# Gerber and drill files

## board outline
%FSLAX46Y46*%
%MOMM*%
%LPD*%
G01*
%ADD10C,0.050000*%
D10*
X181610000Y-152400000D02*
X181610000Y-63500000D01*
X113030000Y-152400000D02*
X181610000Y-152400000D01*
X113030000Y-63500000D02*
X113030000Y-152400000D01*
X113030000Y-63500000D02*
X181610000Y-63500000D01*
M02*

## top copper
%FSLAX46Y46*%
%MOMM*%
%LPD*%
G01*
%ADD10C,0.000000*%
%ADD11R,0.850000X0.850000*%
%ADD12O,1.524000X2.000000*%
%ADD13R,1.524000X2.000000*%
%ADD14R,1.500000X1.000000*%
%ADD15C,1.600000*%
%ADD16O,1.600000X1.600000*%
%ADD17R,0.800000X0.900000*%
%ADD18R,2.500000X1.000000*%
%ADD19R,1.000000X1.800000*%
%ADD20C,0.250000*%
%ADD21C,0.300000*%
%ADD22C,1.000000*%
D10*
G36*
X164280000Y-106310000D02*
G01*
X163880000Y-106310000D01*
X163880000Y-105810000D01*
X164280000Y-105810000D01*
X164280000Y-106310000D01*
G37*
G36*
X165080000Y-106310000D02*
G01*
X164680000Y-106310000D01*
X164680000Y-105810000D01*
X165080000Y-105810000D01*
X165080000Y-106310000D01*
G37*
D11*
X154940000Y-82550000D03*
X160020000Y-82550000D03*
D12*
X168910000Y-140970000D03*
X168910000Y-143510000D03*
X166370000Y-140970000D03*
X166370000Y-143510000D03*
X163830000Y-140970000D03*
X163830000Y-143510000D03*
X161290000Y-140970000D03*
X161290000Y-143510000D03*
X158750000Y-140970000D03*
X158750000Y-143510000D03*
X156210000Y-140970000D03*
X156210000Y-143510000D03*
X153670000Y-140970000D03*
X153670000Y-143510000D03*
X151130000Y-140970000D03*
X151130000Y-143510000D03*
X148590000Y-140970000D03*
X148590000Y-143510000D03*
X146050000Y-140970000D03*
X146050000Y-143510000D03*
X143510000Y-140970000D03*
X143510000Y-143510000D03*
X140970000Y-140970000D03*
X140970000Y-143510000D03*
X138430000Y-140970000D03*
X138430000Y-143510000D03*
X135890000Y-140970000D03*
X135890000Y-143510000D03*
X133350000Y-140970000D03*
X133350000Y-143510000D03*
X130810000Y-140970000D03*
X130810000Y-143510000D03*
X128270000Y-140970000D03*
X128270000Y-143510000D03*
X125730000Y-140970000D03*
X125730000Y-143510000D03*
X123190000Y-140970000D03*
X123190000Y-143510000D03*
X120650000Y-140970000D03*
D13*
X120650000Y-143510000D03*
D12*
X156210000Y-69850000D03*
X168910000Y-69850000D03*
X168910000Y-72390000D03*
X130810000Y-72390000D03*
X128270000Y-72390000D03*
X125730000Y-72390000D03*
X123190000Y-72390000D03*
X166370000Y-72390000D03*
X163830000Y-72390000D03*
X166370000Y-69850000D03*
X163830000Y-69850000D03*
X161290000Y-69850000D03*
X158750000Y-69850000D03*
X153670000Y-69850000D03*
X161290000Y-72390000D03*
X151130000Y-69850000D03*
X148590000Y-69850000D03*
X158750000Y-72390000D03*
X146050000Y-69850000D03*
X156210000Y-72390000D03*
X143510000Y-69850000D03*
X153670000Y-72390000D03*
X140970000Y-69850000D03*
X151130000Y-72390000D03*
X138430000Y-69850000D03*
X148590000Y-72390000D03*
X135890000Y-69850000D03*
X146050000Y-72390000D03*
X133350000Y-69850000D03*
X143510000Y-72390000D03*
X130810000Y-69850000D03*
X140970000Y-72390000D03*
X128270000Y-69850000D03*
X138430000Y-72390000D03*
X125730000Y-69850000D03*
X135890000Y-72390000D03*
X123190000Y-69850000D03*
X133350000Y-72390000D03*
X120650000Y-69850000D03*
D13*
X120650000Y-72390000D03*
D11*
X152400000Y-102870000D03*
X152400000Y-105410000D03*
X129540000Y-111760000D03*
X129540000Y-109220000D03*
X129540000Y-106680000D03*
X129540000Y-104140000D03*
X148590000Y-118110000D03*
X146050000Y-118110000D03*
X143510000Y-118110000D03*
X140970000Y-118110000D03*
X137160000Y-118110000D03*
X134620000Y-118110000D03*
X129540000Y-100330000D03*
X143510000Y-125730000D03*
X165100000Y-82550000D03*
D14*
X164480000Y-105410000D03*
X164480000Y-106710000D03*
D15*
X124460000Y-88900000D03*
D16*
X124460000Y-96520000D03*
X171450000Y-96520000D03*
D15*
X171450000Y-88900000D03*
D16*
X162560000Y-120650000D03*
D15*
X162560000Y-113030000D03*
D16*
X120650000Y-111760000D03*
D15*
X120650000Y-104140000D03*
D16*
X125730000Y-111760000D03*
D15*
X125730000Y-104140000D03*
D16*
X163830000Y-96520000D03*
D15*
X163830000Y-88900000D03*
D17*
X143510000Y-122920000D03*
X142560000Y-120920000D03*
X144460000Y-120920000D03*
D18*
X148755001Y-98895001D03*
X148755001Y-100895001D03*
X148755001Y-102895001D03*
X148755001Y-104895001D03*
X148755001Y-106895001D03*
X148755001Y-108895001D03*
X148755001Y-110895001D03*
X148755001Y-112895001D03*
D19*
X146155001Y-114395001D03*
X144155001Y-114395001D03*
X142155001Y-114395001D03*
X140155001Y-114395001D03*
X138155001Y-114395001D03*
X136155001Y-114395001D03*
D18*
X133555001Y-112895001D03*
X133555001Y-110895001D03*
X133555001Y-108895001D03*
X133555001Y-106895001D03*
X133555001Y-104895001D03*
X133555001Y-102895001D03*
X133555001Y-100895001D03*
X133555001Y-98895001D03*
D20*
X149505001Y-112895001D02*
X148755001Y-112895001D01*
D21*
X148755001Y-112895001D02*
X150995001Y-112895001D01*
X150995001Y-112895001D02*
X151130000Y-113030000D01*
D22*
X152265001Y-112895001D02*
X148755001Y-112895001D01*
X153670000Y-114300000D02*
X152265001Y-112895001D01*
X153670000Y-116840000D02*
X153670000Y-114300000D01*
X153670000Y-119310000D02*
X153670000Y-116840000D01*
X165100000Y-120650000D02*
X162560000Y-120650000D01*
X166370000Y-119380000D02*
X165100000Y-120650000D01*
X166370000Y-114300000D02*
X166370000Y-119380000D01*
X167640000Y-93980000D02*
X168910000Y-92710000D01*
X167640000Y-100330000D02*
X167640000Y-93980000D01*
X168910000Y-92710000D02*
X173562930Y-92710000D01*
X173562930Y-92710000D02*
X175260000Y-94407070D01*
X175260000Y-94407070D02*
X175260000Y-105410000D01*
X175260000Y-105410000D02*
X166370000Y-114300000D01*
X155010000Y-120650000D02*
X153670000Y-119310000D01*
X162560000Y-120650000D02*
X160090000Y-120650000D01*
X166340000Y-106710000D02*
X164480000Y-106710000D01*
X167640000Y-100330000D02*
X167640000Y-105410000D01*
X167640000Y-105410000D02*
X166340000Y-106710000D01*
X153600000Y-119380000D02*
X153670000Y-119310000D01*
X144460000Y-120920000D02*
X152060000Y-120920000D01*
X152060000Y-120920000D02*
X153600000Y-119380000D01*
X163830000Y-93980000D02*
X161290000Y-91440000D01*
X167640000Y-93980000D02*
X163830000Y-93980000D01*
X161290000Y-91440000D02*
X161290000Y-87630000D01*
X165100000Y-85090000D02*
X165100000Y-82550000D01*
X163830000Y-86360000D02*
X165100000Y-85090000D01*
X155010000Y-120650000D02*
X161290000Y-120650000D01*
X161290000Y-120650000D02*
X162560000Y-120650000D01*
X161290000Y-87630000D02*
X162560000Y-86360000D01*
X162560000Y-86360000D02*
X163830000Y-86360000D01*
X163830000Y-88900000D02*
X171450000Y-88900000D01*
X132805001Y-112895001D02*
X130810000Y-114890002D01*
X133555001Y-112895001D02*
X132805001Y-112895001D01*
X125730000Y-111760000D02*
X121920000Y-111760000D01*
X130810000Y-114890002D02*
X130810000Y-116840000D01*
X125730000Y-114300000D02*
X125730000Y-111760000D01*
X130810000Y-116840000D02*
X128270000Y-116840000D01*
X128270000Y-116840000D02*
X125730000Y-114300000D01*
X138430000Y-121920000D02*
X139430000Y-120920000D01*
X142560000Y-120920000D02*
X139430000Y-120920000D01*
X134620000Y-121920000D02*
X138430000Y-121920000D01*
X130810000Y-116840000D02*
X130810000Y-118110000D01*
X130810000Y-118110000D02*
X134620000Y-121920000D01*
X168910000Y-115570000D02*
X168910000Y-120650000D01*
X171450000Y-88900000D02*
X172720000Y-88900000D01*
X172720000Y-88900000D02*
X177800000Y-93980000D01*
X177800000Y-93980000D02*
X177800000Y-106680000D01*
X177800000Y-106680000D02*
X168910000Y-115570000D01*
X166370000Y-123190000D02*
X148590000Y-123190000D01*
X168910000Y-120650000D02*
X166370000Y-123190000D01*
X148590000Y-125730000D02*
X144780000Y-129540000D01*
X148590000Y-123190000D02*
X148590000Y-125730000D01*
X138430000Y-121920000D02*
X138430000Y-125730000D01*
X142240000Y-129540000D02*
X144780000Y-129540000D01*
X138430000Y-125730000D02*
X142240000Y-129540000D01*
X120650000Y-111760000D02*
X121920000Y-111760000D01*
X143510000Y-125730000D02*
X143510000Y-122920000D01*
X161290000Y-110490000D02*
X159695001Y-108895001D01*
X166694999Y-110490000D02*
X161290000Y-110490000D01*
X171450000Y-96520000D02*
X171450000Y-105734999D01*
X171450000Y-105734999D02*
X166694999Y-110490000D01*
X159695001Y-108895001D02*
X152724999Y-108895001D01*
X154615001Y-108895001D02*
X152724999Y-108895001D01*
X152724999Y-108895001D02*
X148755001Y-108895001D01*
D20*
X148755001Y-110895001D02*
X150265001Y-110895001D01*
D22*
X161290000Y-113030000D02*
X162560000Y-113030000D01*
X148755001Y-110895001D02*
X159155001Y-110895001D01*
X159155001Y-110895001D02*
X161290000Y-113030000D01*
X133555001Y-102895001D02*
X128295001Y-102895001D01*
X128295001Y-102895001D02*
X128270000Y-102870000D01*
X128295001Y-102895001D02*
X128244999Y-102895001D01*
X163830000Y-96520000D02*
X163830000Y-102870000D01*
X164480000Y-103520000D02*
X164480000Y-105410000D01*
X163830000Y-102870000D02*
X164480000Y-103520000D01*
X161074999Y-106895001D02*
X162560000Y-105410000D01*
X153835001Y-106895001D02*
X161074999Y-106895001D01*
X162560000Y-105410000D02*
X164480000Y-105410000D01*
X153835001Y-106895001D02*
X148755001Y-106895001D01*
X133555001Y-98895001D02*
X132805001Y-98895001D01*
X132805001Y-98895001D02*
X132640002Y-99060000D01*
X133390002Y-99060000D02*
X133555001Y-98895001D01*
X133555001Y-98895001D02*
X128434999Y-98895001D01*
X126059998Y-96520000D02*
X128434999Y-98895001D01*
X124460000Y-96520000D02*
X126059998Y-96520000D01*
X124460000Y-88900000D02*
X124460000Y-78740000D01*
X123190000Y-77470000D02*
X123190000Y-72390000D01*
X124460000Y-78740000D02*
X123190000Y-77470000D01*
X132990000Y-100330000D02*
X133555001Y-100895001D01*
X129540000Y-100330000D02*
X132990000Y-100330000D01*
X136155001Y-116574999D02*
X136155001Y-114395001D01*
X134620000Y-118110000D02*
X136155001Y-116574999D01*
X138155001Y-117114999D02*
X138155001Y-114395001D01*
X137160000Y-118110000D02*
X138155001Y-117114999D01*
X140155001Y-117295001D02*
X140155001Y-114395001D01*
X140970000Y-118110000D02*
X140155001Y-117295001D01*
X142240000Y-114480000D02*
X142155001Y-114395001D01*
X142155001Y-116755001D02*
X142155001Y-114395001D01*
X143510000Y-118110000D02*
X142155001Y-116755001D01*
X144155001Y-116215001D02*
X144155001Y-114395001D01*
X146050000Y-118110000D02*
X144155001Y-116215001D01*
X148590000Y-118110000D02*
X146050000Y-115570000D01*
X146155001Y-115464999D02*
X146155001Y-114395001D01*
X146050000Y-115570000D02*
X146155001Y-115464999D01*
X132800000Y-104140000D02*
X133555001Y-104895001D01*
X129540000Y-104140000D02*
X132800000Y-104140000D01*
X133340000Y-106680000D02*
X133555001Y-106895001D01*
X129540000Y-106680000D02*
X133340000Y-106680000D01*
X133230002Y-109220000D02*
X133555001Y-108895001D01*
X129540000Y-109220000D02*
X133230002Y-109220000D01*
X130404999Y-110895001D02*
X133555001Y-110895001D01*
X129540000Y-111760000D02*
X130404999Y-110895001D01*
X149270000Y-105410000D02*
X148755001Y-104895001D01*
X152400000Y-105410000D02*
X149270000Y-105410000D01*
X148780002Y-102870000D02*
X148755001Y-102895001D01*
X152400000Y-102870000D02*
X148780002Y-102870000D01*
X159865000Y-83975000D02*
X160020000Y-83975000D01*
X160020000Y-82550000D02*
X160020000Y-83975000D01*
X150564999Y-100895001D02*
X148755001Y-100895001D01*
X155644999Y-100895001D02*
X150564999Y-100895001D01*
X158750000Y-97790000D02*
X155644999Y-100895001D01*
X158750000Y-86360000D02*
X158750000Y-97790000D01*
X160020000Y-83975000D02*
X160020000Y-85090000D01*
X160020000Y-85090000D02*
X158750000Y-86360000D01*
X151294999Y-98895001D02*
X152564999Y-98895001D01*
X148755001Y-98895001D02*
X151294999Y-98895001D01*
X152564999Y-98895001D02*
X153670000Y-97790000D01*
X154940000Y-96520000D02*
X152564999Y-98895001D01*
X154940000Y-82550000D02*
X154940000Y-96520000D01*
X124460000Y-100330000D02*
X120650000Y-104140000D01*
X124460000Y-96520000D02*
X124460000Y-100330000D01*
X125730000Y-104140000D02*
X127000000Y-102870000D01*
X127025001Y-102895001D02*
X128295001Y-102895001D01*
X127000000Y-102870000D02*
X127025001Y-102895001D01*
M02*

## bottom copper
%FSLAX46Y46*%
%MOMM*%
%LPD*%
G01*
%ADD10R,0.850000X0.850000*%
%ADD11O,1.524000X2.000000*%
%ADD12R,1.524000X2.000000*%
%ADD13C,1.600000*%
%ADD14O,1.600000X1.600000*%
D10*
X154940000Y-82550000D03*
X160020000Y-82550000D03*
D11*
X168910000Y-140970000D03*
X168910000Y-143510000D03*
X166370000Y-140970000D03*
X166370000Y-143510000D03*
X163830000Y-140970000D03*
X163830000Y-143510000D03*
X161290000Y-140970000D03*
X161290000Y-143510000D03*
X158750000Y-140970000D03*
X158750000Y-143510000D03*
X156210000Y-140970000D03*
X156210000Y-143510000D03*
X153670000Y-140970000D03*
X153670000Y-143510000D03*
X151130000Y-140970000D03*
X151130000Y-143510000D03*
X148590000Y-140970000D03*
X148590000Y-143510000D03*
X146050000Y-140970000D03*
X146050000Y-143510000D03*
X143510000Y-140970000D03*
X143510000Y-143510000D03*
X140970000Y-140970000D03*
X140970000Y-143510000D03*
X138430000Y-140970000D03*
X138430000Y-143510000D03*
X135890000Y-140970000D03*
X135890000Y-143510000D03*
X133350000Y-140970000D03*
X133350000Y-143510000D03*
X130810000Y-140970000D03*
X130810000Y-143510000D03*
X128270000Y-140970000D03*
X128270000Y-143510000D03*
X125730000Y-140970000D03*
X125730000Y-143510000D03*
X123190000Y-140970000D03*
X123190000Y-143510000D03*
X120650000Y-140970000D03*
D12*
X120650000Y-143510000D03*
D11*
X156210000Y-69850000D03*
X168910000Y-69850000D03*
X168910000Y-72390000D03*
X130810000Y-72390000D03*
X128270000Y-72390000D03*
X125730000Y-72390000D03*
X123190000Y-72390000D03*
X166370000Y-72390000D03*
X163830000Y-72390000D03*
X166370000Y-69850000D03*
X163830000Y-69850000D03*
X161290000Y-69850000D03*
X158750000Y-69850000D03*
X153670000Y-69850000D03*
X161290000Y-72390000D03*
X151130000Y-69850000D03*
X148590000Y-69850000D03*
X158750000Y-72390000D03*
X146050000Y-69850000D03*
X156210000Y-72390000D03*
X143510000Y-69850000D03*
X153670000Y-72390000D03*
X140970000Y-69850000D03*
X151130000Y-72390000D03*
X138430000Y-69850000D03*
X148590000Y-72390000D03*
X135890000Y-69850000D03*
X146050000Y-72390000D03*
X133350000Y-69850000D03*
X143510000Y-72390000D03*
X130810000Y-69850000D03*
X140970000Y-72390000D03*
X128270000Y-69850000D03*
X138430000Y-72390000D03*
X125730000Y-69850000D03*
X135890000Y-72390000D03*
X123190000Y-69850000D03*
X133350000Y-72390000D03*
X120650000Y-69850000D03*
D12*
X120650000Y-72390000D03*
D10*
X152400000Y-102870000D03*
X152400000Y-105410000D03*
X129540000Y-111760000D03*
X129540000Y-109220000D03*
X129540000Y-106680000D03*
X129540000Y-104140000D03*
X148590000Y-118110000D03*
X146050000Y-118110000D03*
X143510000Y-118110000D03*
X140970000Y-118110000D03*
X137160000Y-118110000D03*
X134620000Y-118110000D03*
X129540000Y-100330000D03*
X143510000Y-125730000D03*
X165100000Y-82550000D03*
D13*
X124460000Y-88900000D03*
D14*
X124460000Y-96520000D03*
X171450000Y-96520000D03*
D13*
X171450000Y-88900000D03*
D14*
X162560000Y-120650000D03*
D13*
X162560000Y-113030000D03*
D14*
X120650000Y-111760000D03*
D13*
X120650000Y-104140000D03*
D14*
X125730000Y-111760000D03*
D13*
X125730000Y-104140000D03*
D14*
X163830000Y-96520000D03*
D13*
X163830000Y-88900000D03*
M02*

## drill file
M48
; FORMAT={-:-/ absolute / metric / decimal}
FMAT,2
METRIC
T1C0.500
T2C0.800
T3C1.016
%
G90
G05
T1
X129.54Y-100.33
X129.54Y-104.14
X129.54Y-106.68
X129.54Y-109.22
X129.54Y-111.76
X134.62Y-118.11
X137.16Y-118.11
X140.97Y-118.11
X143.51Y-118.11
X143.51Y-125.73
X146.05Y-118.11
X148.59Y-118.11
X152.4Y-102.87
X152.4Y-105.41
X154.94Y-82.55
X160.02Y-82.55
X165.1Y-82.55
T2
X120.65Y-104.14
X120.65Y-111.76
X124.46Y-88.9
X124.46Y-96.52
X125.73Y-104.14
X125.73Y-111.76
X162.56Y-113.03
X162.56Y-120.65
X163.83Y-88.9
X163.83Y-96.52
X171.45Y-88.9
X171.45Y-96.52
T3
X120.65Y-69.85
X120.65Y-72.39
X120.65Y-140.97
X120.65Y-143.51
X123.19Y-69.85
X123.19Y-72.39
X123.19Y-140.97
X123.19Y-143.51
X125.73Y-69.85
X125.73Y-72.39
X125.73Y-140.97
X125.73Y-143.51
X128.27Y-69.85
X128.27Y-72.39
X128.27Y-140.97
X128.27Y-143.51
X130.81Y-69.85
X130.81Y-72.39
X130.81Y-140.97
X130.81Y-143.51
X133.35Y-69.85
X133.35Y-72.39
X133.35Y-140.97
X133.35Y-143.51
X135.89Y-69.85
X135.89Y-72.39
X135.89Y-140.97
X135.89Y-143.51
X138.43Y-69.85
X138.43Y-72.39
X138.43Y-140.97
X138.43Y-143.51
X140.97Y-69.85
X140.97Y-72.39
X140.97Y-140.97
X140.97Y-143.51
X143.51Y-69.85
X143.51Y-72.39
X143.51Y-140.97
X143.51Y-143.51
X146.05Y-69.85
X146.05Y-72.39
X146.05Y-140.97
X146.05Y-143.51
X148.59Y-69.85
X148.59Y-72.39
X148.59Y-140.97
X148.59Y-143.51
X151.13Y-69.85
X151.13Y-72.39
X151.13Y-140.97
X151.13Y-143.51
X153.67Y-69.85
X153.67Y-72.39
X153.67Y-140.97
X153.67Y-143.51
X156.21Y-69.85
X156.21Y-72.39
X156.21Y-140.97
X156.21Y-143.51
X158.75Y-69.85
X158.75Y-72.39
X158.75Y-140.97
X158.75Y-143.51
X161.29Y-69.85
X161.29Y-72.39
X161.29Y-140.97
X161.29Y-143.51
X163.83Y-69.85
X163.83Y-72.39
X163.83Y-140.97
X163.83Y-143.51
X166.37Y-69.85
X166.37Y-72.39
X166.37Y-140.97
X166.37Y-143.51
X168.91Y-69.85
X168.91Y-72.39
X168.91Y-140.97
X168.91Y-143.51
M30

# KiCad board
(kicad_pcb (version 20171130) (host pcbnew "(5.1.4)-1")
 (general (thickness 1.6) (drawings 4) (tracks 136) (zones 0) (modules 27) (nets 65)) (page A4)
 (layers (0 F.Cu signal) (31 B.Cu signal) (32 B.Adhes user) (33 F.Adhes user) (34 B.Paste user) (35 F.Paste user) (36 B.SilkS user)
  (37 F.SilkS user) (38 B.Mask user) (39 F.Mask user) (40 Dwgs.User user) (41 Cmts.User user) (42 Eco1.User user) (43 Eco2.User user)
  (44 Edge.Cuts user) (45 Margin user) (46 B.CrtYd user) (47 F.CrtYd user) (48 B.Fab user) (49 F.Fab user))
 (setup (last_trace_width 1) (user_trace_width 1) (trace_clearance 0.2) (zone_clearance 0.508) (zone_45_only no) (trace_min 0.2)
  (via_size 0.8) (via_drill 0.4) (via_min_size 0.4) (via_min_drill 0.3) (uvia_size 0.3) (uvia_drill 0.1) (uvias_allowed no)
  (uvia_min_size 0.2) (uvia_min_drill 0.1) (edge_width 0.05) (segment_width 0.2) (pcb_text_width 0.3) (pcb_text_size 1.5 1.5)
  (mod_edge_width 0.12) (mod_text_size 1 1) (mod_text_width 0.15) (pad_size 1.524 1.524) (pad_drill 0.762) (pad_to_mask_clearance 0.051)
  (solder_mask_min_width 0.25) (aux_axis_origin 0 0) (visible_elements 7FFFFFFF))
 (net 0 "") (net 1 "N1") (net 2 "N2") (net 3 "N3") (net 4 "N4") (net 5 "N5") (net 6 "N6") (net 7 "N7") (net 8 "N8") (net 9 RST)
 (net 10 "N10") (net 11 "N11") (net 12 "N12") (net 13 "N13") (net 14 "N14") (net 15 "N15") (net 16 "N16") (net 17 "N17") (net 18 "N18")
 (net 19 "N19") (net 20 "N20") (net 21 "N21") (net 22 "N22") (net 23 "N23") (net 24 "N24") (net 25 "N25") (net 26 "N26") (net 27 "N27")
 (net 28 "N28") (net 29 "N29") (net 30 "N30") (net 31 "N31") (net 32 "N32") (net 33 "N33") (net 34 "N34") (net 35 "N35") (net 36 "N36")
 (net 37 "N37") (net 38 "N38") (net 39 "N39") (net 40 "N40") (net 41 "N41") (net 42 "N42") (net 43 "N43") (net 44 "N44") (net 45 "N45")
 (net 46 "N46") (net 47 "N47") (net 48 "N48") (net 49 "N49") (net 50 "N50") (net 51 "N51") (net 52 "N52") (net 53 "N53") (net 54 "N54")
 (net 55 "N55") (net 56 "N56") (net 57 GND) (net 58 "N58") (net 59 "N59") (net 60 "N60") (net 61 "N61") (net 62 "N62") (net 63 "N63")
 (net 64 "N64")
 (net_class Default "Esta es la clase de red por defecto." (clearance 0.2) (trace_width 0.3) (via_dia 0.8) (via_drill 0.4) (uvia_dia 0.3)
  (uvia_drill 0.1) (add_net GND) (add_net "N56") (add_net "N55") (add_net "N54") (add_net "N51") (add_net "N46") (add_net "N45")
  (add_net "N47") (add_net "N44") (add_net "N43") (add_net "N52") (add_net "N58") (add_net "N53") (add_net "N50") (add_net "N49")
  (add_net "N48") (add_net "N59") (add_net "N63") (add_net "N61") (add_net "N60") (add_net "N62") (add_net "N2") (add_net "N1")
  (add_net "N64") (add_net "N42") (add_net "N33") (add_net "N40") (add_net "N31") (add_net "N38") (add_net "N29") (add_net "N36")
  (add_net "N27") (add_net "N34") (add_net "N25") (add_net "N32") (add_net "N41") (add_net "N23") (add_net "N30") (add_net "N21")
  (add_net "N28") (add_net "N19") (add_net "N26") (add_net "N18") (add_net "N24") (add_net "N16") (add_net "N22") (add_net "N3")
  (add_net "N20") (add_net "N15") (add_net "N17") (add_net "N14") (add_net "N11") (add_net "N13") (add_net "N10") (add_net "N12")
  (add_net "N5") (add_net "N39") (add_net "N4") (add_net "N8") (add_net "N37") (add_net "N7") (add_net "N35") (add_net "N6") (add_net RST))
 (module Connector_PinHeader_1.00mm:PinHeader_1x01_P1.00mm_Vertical (layer F.Cu) (at 154.94 82.55)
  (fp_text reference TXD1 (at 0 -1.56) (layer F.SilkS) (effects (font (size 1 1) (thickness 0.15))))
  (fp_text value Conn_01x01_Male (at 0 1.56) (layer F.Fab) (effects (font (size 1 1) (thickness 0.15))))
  (pad 1 thru_hole rect (at 0 0) (size 0.85 0.85) (drill 0.5) (layers *.Cu *.Mask) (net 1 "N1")))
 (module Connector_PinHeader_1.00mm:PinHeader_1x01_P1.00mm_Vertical (layer F.Cu) (at 160.02 82.55)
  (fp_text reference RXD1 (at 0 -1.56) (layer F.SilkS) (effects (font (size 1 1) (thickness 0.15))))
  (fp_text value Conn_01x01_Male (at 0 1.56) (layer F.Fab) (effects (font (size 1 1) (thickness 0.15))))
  (pad 1 thru_hole rect (at 0 0) (size 0.85 0.85) (drill 0.5) (layers *.Cu *.Mask) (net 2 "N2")))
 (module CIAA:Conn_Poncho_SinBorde (layer F.Cu) (at 120.65 72.39 90)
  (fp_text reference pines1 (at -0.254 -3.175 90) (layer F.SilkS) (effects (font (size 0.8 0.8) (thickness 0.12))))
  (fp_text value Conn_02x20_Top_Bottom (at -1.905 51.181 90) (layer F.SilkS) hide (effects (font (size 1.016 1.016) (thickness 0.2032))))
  (pad 80 thru_hole oval (at -68.58 48.26) (size 1.524 2) (drill 1.016) (layers *.Cu *.Mask F.SilkS))
  (pad 79 thru_hole oval (at -71.12 48.26) (size 1.524 2) (drill 1.016) (layers *.Cu *.Mask F.SilkS))
  (pad 78 thru_hole oval (at -68.58 45.72) (size 1.524 2) (drill 1.016) (layers *.Cu *.Mask F.SilkS))
  (pad 77 thru_hole oval (at -71.12 45.72) (size 1.524 2) (drill 1.016) (layers *.Cu *.Mask F.SilkS))
  (pad 76 thru_hole oval (at -68.58 43.18) (size 1.524 2) (drill 1.016) (layers *.Cu *.Mask F.SilkS))
  (pad 75 thru_hole oval (at -71.12 43.18) (size 1.524 2) (drill 1.016) (layers *.Cu *.Mask F.SilkS))
  (pad 74 thru_hole oval (at -68.58 40.64) (size 1.524 2) (drill 1.016) (layers *.Cu *.Mask F.SilkS))
  (pad 73 thru_hole oval (at -71.12 40.64) (size 1.524 2) (drill 1.016) (layers *.Cu *.Mask F.SilkS))
  (pad 72 thru_hole oval (at -68.58 38.1) (size 1.524 2) (drill 1.016) (layers *.Cu *.Mask F.SilkS))
  (pad 71 thru_hole oval (at -71.12 38.1) (size 1.524 2) (drill 1.016) (layers *.Cu *.Mask F.SilkS))
  (pad 70 thru_hole oval (at -68.58 35.56) (size 1.524 2) (drill 1.016) (layers *.Cu *.Mask F.SilkS))
  (pad 69 thru_hole oval (at -71.12 35.56) (size 1.524 2) (drill 1.016) (layers *.Cu *.Mask F.SilkS))
  (pad 68 thru_hole oval (at -68.58 33.02) (size 1.524 2) (drill 1.016) (layers *.Cu *.Mask F.SilkS))
  (pad 67 thru_hole oval (at -71.12 33.02) (size 1.524 2) (drill 1.016) (layers *.Cu *.Mask F.SilkS))
  (pad 66 thru_hole oval (at -68.58 30.48) (size 1.524 2) (drill 1.016) (layers *.Cu *.Mask F.SilkS))
  (pad 65 thru_hole oval (at -71.12 30.48) (size 1.524 2) (drill 1.016) (layers *.Cu *.Mask F.SilkS))
  (pad 64 thru_hole oval (at -68.58 27.94) (size 1.524 2) (drill 1.016) (layers *.Cu *.Mask F.SilkS))
  (pad 63 thru_hole oval (at -71.12 27.94) (size 1.524 2) (drill 1.016) (layers *.Cu *.Mask F.SilkS))
  (pad 62 thru_hole oval (at -68.58 25.4) (size 1.524 2) (drill 1.016) (layers *.Cu *.Mask F.SilkS))
  (pad 61 thru_hole oval (at -71.12 25.4) (size 1.524 2) (drill 1.016) (layers *.Cu *.Mask F.SilkS))
  (pad 60 thru_hole oval (at -68.58 22.86) (size 1.524 2) (drill 1.016) (layers *.Cu *.Mask F.SilkS))
  (pad 59 thru_hole oval (at -71.12 22.86) (size 1.524 2) (drill 1.016) (layers *.Cu *.Mask F.SilkS))
  (pad 58 thru_hole oval (at -68.58 20.32) (size 1.524 2) (drill 1.016) (layers *.Cu *.Mask F.SilkS))
  (pad 57 thru_hole oval (at -71.12 20.32) (size 1.524 2) (drill 1.016) (layers *.Cu *.Mask F.SilkS))
  (pad 56 thru_hole oval (at -68.58 17.78) (size 1.524 2) (drill 1.016) (layers *.Cu *.Mask F.SilkS))
  (pad 55 thru_hole oval (at -71.12 17.78) (size 1.524 2) (drill 1.016) (layers *.Cu *.Mask F.SilkS))
  (pad 54 thru_hole oval (at -68.58 15.24) (size 1.524 2) (drill 1.016) (layers *.Cu *.Mask F.SilkS))
  (pad 53 thru_hole oval (at -71.12 15.24) (size 1.524 2) (drill 1.016) (layers *.Cu *.Mask F.SilkS))
  (pad 52 thru_hole oval (at -68.58 12.7) (size 1.524 2) (drill 1.016) (layers *.Cu *.Mask F.SilkS))
  (pad 51 thru_hole oval (at -71.12 12.7) (size 1.524 2) (drill 1.016) (layers *.Cu *.Mask F.SilkS))
  (pad 50 thru_hole oval (at -68.58 10.16) (size 1.524 2) (drill 1.016) (layers *.Cu *.Mask F.SilkS))
  (pad 49 thru_hole oval (at -71.12 10.16) (size 1.524 2) (drill 1.016) (layers *.Cu *.Mask F.SilkS))
  (pad 48 thru_hole oval (at -68.58 7.62) (size 1.524 2) (drill 1.016) (layers *.Cu *.Mask F.SilkS))
  (pad 47 thru_hole oval (at -71.12 7.62) (size 1.524 2) (drill 1.016) (layers *.Cu *.Mask F.SilkS))
  (pad 46 thru_hole oval (at -68.58 5.08) (size 1.524 2) (drill 1.016) (layers *.Cu *.Mask F.SilkS))
  (pad 45 thru_hole oval (at -71.12 5.08) (size 1.524 2) (drill 1.016) (layers *.Cu *.Mask F.SilkS))
  (pad 44 thru_hole oval (at -68.58 2.54) (size 1.524 2) (drill 1.016) (layers *.Cu *.Mask F.SilkS))
  (pad 43 thru_hole oval (at -71.12 2.54) (size 1.524 2) (drill 1.016) (layers *.Cu *.Mask F.SilkS))
  (pad 42 thru_hole oval (at -68.58 0) (size 1.524 2) (drill 1.016) (layers *.Cu *.Mask F.SilkS))
  (pad 41 thru_hole rect (at -71.12 0) (size 1.524 2) (drill 1.016) (layers *.Cu *.Mask F.SilkS))
  (pad 30 thru_hole oval (at 2.54 35.56) (size 1.524 2) (drill 1.016) (layers *.Cu *.Mask F.SilkS) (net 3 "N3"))
  (pad 40 thru_hole oval (at 2.54 48.26) (size 1.524 2) (drill 1.016) (layers *.Cu *.Mask F.SilkS) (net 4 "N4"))
  (pad 39 thru_hole oval (at 0 48.26) (size 1.524 2) (drill 1.016) (layers *.Cu *.Mask F.SilkS) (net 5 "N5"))
  (pad 9 thru_hole oval (at 0 10.16) (size 1.524 2) (drill 1.016) (layers *.Cu *.Mask F.SilkS) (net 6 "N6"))
  (pad 7 thru_hole oval (at 0 7.62) (size 1.524 2) (drill 1.016) (layers *.Cu *.Mask F.SilkS) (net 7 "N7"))
  (pad 5 thru_hole oval (at 0 5.08) (size 1.524 2) (drill 1.016) (layers *.Cu *.Mask F.SilkS) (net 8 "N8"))
  (pad 3 thru_hole oval (at 0 2.54) (size 1.524 2) (drill 1.016) (layers *.Cu *.Mask F.SilkS) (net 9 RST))
  (pad 37 thru_hole oval (at 0 45.72) (size 1.524 2) (drill 1.016) (layers *.Cu *.Mask F.SilkS) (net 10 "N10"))
  (pad 35 thru_hole oval (at 0 43.18) (size 1.524 2) (drill 1.016) (layers *.Cu *.Mask F.SilkS) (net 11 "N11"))
  (pad 38 thru_hole oval (at 2.54 45.72) (size 1.524 2) (drill 1.016) (layers *.Cu *.Mask F.SilkS) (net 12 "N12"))
  (pad 36 thru_hole oval (at 2.54 43.18) (size 1.524 2) (drill 1.016) (layers *.Cu *.Mask F.SilkS) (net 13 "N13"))
  (pad 34 thru_hole oval (at 2.54 40.64) (size 1.524 2) (drill 1.016) (layers *.Cu *.Mask F.SilkS) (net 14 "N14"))
  (pad 32 thru_hole oval (at 2.54 38.1) (size 1.524 2) (drill 1.016) (layers *.Cu *.Mask F.SilkS) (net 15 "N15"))
  (pad 28 thru_hole oval (at 2.54 33.02) (size 1.524 2) (drill 1.016) (layers *.Cu *.Mask F.SilkS) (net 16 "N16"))
  (pad 33 thru_hole oval (at 0 40.64) (size 1.524 2) (drill 1.016) (layers *.Cu *.Mask F.SilkS) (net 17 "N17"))
  (pad 26 thru_hole oval (at 2.54 30.48) (size 1.524 2) (drill 1.016) (layers *.Cu *.Mask F.SilkS) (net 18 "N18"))
  (pad 24 thru_hole oval (at 2.54 27.94) (size 1.524 2) (drill 1.016) (layers *.Cu *.Mask F.SilkS) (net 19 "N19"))
  (pad 31 thru_hole oval (at 0 38.1) (size 1.524 2) (drill 1.016) (layers *.Cu *.Mask F.SilkS) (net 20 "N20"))
  (pad 22 thru_hole oval (at 2.54 25.4) (size 1.524 2) (drill 1.016) (layers *.Cu *.Mask F.SilkS) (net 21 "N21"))
  (pad 29 thru_hole oval (at 0 35.56) (size 1.524 2) (drill 1.016) (layers *.Cu *.Mask F.SilkS) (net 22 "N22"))
  (pad 20 thru_hole oval (at 2.54 22.86) (size 1.524 2) (drill 1.016) (layers *.Cu *.Mask F.SilkS) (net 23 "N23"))
  (pad 27 thru_hole oval (at 0 33.02) (size 1.524 2) (drill 1.016) (layers *.Cu *.Mask F.SilkS) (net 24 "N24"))
  (pad 18 thru_hole oval (at 2.54 20.32) (size 1.524 2) (drill 1.016) (layers *.Cu *.Mask F.SilkS) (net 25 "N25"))
  (pad 25 thru_hole oval (at 0 30.48) (size 1.524 2) (drill 1.016) (layers *.Cu *.Mask F.SilkS) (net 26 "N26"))
  (pad 16 thru_hole oval (at 2.54 17.78) (size 1.524 2) (drill 1.016) (layers *.Cu *.Mask F.SilkS) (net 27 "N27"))
  (pad 23 thru_hole oval (at 0 27.94) (size 1.524 2) (drill 1.016) (layers *.Cu *.Mask F.SilkS) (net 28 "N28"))
  (pad 14 thru_hole oval (at 2.54 15.24) (size 1.524 2) (drill 1.016) (layers *.Cu *.Mask F.SilkS) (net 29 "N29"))
  (pad 21 thru_hole oval (at 0 25.4) (size 1.524 2) (drill 1.016) (layers *.Cu *.Mask F.SilkS) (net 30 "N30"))
  (pad 12 thru_hole oval (at 2.54 12.7) (size 1.524 2) (drill 1.016) (layers *.Cu *.Mask F.SilkS) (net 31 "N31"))
  (pad 19 thru_hole oval (at 0 22.86) (size 1.524 2) (drill 1.016) (layers *.Cu *.Mask F.SilkS) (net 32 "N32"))
  (pad 10 thru_hole oval (at 2.54 10.16) (size 1.524 2) (drill 1.016) (layers *.Cu *.Mask F.SilkS) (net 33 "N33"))
  (pad 17 thru_hole oval (at 0 20.32) (size 1.524 2) (drill 1.016) (layers *.Cu *.Mask F.SilkS) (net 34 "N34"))
  (pad 8 thru_hole oval (at 2.54 7.62) (size 1.524 2) (drill 1.016) (layers *.Cu *.Mask F.SilkS) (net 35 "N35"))
  (pad 15 thru_hole oval (at 0 17.78) (size 1.524 2) (drill 1.016) (layers *.Cu *.Mask F.SilkS) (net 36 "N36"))
  (pad 6 thru_hole oval (at 2.54 5.08) (size 1.524 2) (drill 1.016) (layers *.Cu *.Mask F.SilkS) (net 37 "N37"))
  (pad 13 thru_hole oval (at 0 15.24) (size 1.524 2) (drill 1.016) (layers *.Cu *.Mask F.SilkS) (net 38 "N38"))
  (pad 4 thru_hole oval (at 2.54 2.54) (size 1.524 2) (drill 1.016) (layers *.Cu *.Mask F.SilkS) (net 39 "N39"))
  (pad 11 thru_hole oval (at 0 12.7) (size 1.524 2) (drill 1.016) (layers *.Cu *.Mask F.SilkS) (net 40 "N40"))
  (pad 2 thru_hole oval (at 2.54 0) (size 1.524 2) (drill 1.016) (layers *.Cu *.Mask F.SilkS) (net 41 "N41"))
  (pad 1 thru_hole rect (at 0 0) (size 1.524 2) (drill 1.016) (layers *.Cu *.Mask F.SilkS) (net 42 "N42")))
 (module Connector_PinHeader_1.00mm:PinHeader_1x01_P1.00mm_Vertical (layer F.Cu) (at 152.4 102.87)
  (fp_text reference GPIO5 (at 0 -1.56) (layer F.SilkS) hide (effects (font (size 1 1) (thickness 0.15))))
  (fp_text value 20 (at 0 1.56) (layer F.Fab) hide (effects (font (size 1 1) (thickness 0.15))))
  (pad 1 thru_hole rect (at 0 0) (size 0.85 0.85) (drill 0.5) (layers *.Cu *.Mask) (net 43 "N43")))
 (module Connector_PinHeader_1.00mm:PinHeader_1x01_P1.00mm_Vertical (layer F.Cu) (at 152.4 105.41)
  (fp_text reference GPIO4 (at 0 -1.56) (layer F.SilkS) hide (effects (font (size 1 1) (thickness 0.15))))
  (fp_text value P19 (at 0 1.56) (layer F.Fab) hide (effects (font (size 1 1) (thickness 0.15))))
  (pad 1 thru_hole rect (at 0 0) (size 0.85 0.85) (drill 0.5) (layers *.Cu *.Mask) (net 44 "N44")))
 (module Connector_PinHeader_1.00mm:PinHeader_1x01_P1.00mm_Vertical (layer F.Cu) (at 129.54 111.76)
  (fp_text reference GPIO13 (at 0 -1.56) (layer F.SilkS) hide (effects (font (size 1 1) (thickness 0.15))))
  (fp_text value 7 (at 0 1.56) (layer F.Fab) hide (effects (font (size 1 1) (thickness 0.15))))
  (pad 1 thru_hole rect (at 0 0) (size 0.85 0.85) (drill 0.5) (layers *.Cu *.Mask) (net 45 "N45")))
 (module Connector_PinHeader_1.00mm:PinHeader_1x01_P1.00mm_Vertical (layer F.Cu) (at 129.54 109.22)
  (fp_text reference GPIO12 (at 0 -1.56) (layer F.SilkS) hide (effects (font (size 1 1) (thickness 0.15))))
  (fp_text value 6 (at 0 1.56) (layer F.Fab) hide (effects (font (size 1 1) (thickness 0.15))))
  (pad 1 thru_hole rect (at 0 0) (size 0.85 0.85) (drill 0.5) (layers *.Cu *.Mask) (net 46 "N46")))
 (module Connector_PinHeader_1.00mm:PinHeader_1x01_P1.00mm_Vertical (layer F.Cu) (at 129.54 106.68)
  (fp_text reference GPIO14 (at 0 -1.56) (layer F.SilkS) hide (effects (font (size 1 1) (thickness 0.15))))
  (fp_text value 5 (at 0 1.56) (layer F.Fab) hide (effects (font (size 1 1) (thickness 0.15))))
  (pad 1 thru_hole rect (at 0 0) (size 0.85 0.85) (drill 0.5) (layers *.Cu *.Mask) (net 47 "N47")))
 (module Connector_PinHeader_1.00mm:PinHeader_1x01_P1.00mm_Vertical (layer F.Cu) (at 129.54 104.14)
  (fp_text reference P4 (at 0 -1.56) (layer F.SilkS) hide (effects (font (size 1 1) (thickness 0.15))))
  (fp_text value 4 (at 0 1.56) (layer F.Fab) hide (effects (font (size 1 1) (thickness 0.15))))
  (pad 1 thru_hole rect (at 0 0) (size 0.85 0.85) (drill 0.5) (layers *.Cu *.Mask) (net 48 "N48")))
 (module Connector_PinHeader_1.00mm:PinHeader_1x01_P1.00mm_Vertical (layer F.Cu) (at 148.59 118.11)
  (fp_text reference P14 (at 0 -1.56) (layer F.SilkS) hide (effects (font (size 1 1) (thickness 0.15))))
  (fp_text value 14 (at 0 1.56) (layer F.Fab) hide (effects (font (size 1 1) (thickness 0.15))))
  (pad 1 thru_hole rect (at 0 0) (size 0.85 0.85) (drill 0.5) (layers *.Cu *.Mask) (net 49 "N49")))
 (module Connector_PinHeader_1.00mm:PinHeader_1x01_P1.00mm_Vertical (layer F.Cu) (at 146.05 118.11)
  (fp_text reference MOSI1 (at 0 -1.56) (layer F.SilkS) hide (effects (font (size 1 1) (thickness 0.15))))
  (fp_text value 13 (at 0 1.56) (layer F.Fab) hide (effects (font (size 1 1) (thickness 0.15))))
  (pad 1 thru_hole rect (at 0 0) (size 0.85 0.85) (drill 0.5) (layers *.Cu *.Mask) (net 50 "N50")))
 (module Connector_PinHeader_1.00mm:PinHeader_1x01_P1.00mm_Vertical (layer F.Cu) (at 143.51 118.11)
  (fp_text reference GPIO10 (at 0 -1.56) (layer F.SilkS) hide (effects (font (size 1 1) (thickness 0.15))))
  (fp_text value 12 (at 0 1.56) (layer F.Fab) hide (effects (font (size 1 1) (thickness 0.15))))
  (pad 1 thru_hole rect (at 0 0) (size 0.85 0.85) (drill 0.5) (layers *.Cu *.Mask) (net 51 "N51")))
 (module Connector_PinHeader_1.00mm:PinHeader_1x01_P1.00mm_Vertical (layer F.Cu) (at 140.97 118.11)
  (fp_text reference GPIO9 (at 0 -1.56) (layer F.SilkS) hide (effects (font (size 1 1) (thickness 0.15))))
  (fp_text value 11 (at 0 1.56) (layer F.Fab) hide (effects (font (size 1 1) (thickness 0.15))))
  (pad 1 thru_hole rect (at 0 0) (size 0.85 0.85) (drill 0.5) (layers *.Cu *.Mask) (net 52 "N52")))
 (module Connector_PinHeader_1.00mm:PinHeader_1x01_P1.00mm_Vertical (layer F.Cu) (at 137.16 118.11)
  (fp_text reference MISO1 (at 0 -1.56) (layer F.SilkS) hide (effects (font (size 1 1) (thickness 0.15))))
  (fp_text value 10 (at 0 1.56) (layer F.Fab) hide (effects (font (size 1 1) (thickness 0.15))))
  (pad 1 thru_hole rect (at 0 0) (size 0.85 0.85) (drill 0.5) (layers *.Cu *.Mask) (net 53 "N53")))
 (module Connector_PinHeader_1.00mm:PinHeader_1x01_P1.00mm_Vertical (layer F.Cu) (at 134.62 118.11)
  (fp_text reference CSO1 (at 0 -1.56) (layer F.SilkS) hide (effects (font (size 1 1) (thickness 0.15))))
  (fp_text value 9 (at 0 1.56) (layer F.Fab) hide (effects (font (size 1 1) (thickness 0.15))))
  (pad 1 thru_hole rect (at 0 0) (size 0.85 0.85) (drill 0.5) (layers *.Cu *.Mask) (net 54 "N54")))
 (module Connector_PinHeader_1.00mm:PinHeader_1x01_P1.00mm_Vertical (layer F.Cu) (at 129.54 100.33)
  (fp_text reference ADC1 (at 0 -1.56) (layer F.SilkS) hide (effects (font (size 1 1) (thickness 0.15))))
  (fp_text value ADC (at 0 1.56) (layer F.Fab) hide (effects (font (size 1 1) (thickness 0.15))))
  (pad 1 thru_hole rect (at 0 0) (size 0.85 0.85) (drill 0.5) (layers *.Cu *.Mask) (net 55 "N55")))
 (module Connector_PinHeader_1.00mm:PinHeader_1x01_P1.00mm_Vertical (layer F.Cu) (at 143.51 125.73 180)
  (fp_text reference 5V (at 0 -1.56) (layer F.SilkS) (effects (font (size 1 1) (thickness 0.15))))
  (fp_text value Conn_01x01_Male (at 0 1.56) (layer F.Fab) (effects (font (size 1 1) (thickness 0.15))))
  (pad 1 thru_hole rect (at 0 0 180) (size 0.85 0.85) (drill 0.5) (layers *.Cu *.Mask) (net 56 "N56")))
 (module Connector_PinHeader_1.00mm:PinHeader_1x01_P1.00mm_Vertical (layer F.Cu) (at 165.1 82.55)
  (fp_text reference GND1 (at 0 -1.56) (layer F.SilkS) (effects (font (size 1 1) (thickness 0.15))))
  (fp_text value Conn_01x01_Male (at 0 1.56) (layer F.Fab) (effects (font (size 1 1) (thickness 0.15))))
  (pad 1 thru_hole rect (at 0 0) (size 0.85 0.85) (drill 0.5) (layers *.Cu *.Mask) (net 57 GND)))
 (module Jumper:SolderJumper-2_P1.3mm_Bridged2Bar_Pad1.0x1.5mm (layer F.Cu) (at 164.48 106.06 90)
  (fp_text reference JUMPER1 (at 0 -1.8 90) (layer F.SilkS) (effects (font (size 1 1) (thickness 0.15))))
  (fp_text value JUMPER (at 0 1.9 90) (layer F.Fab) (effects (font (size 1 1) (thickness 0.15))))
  (fp_poly (pts (xy -0.25 -0.6) (xy 0.25 -0.6) (xy 0.25 -0.2) (xy -0.25 -0.2)) (layer F.Cu) (width 0))
  (fp_poly (pts (xy -0.25 0.2) (xy 0.25 0.2) (xy 0.25 0.6) (xy -0.25 0.6)) (layer F.Cu) (width 0))
  (pad 2 smd rect (at 0.65 0 90) (size 1 1.5) (layers F.Cu F.Mask) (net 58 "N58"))
  (pad 1 smd rect (at -0.65 0 90) (size 1 1.5) (layers F.Cu F.Mask) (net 57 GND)))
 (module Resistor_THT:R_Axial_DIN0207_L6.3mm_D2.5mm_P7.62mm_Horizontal (layer F.Cu) (at 124.46 88.9 270)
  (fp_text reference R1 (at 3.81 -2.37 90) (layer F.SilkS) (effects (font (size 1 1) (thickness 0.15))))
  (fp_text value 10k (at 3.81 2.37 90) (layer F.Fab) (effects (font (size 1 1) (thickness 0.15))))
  (pad 1 thru_hole circle (at 0 0 270) (size 1.6 1.6) (drill 0.8) (layers *.Cu *.Mask) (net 9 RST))
  (pad 2 thru_hole oval (at 7.62 0 270) (size 1.6 1.6) (drill 0.8) (layers *.Cu *.Mask) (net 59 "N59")))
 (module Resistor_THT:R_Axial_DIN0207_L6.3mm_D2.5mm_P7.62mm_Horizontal (layer F.Cu) (at 171.45 88.9 270)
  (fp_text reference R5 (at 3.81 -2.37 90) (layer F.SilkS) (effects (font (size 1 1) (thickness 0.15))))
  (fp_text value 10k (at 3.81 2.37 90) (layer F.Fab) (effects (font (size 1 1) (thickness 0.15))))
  (pad 2 thru_hole oval (at 7.62 0 270) (size 1.6 1.6) (drill 0.8) (layers *.Cu *.Mask) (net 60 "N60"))
  (pad 1 thru_hole circle (at 0 0 270) (size 1.6 1.6) (drill 0.8) (layers *.Cu *.Mask) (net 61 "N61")))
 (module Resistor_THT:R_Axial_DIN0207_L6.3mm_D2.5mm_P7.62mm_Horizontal (layer F.Cu) (at 162.56 113.03 270)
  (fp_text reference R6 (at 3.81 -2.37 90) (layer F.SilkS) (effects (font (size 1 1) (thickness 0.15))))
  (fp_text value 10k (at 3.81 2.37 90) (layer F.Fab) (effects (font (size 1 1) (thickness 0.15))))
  (pad 2 thru_hole oval (at 7.62 0 270) (size 1.6 1.6) (drill 0.8) (layers *.Cu *.Mask) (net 57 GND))
  (pad 1 thru_hole circle (at 0 0 270) (size 1.6 1.6) (drill 0.8) (layers *.Cu *.Mask) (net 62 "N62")))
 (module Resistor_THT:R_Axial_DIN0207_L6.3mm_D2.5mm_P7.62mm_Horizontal (layer F.Cu) (at 120.65 104.14 270)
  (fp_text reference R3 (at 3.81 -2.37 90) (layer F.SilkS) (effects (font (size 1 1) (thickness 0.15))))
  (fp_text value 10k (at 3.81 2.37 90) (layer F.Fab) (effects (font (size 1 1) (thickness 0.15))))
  (pad 2 thru_hole oval (at 7.62 0 270) (size 1.6 1.6) (drill 0.8) (layers *.Cu *.Mask) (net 61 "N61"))
  (pad 1 thru_hole circle (at 0 0 270) (size 1.6 1.6) (drill 0.8) (layers *.Cu *.Mask) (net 59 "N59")))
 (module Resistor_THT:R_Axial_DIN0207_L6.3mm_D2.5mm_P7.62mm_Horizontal (layer F.Cu) (at 125.73 104.14 270)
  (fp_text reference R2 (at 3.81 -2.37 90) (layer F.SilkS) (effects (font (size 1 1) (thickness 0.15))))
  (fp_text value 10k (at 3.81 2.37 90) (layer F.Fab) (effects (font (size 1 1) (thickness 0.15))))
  (pad 2 thru_hole oval (at 7.62 0 270) (size 1.6 1.6) (drill 0.8) (layers *.Cu *.Mask) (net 61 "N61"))
  (pad 1 thru_hole circle (at 0 0 270) (size 1.6 1.6) (drill 0.8) (layers *.Cu *.Mask) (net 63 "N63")))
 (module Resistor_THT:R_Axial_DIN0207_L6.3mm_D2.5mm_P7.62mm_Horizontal (layer F.Cu) (at 163.83 88.9 270)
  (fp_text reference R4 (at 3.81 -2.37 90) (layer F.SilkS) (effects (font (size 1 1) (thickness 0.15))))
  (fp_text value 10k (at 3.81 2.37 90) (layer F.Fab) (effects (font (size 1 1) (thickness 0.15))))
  (pad 2 thru_hole oval (at 7.62 0 270) (size 1.6 1.6) (drill 0.8) (layers *.Cu *.Mask) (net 58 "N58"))
  (pad 1 thru_hole circle (at 0 0 270) (size 1.6 1.6) (drill 0.8) (layers *.Cu *.Mask) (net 61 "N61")))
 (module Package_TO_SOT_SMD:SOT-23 (layer F.Cu) (at 143.51 121.92 270)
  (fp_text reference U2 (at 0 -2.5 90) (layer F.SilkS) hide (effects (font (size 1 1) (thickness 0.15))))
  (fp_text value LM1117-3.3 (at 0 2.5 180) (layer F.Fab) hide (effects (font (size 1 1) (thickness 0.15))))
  (pad 3 smd rect (at 1 0 270) (size 0.9 0.8) (layers F.Cu F.Paste F.Mask) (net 56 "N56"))
  (pad 2 smd rect (at -1 0.95 270) (size 0.9 0.8) (layers F.Cu F.Paste F.Mask) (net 61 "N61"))
  (pad 1 smd rect (at -1 -0.95 270) (size 0.9 0.8) (layers F.Cu F.Paste F.Mask) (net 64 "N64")))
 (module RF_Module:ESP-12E (layer F.Cu) (at 141.155001 102.395001)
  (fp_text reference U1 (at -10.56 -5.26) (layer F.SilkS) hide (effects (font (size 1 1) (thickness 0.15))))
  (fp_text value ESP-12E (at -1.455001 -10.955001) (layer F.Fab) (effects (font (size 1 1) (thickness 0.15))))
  (pad 22 smd rect (at 7.6 -3.5) (size 2.5 1) (layers F.Cu F.Paste F.Mask) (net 1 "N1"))
  (pad 21 smd rect (at 7.6 -1.5) (size 2.5 1) (layers F.Cu F.Paste F.Mask) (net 2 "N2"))
  (pad 20 smd rect (at 7.6 0.5) (size 2.5 1) (layers F.Cu F.Paste F.Mask) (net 43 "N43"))
  (pad 19 smd rect (at 7.6 2.5) (size 2.5 1) (layers F.Cu F.Paste F.Mask) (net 44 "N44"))
  (pad 18 smd rect (at 7.6 4.5) (size 2.5 1) (layers F.Cu F.Paste F.Mask) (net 58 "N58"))
  (pad 17 smd rect (at 7.6 6.5) (size 2.5 1) (layers F.Cu F.Paste F.Mask) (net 60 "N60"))
  (pad 16 smd rect (at 7.6 8.5) (size 2.5 1) (layers F.Cu F.Paste F.Mask) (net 62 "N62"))
  (pad 15 smd rect (at 7.6 10.5) (size 2.5 1) (layers F.Cu F.Paste F.Mask) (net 57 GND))
  (pad 14 smd rect (at 5 12) (size 1 1.8) (layers F.Cu F.Paste F.Mask) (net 49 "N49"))
  (pad 13 smd rect (at 3 12) (size 1 1.8) (layers F.Cu F.Paste F.Mask) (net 50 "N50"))
  (pad 12 smd rect (at 1 12) (size 1 1.8) (layers F.Cu F.Paste F.Mask) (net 51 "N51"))
  (pad 11 smd rect (at -1 12) (size 1 1.8) (layers F.Cu F.Paste F.Mask) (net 52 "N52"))
  (pad 10 smd rect (at -3 12) (size 1 1.8) (layers F.Cu F.Paste F.Mask) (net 53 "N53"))
  (pad 9 smd rect (at -5 12) (size 1 1.8) (layers F.Cu F.Paste F.Mask) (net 54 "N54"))
  (pad 8 smd rect (at -7.6 10.5) (size 2.5 1) (layers F.Cu F.Paste F.Mask) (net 61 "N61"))
  (pad 7 smd rect (at -7.6 8.5) (size 2.5 1) (layers F.Cu F.Paste F.Mask) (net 45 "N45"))
  (pad 6 smd rect (at -7.6 6.5) (size 2.5 1) (layers F.Cu F.Paste F.Mask) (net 46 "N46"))
  (pad 5 smd rect (at -7.6 4.5) (size 2.5 1) (layers F.Cu F.Paste F.Mask) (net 47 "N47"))
  (pad 4 smd rect (at -7.6 2.5) (size 2.5 1) (layers F.Cu F.Paste F.Mask) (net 48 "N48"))
  (pad 3 smd rect (at -7.6 0.5) (size 2.5 1) (layers F.Cu F.Paste F.Mask) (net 63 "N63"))
  (pad 2 smd rect (at -7.6 -1.5) (size 2.5 1) (layers F.Cu F.Paste F.Mask) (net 55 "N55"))
  (pad 1 smd rect (at -7.6 -3.5) (size 2.5 1) (layers F.Cu F.Paste F.Mask) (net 59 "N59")))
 (gr_line (start 181.61 152.4) (end 181.61 63.5) (layer Edge.Cuts) (width 0.05))
 (gr_line (start 113.03 152.4) (end 181.61 152.4) (layer Edge.Cuts) (width 0.05))
 (gr_line (start 113.03 63.5) (end 113.03 152.4) (layer Edge.Cuts) (width 0.05))
 (gr_line (start 113.03 63.5) (end 181.61 63.5) (layer Edge.Cuts) (width 0.05))
 (segment (start 149.505001 112.895001) (end 148.755001 112.895001) (width 0.25) (layer F.Cu) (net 57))
 (segment (start 148.755001 112.895001) (end 150.995001 112.895001) (width 0.3) (layer F.Cu) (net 57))
 (segment (start 150.995001 112.895001) (end 151.13 113.03) (width 0.3) (layer F.Cu) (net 57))
 (segment (start 152.265001 112.895001) (end 148.755001 112.895001) (width 1) (layer F.Cu) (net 57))
 (segment (start 153.67 114.3) (end 152.265001 112.895001) (width 1) (layer F.Cu) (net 57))
 (segment (start 153.67 116.84) (end 153.67 114.3) (width 1) (layer F.Cu) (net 57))
 (segment (start 153.67 119.31) (end 153.67 116.84) (width 1) (layer F.Cu) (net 57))
 (segment (start 165.1 120.65) (end 162.56 120.65) (width 1) (layer F.Cu) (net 57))
 (segment (start 166.37 119.38) (end 165.1 120.65) (width 1) (layer F.Cu) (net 57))
 (segment (start 166.37 114.3) (end 166.37 119.38) (width 1) (layer F.Cu) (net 57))
 (segment (start 167.64 93.98) (end 168.91 92.71) (width 1) (layer F.Cu) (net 57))
 (segment (start 167.64 100.33) (end 167.64 93.98) (width 1) (layer F.Cu) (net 57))
 (segment (start 168.91 92.71) (end 173.56293 92.71) (width 1) (layer F.Cu) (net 57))
 (segment (start 173.56293 92.71) (end 175.26 94.40707) (width 1) (layer F.Cu) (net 57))
 (segment (start 175.26 94.40707) (end 175.26 105.41) (width 1) (layer F.Cu) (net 57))
 (segment (start 175.26 105.41) (end 166.37 114.3) (width 1) (layer F.Cu) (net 57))
 (segment (start 155.01 120.65) (end 153.67 119.31) (width 1) (layer F.Cu) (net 57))
 (segment (start 162.56 120.65) (end 160.09 120.65) (width 1) (layer F.Cu) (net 57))
 (segment (start 166.34 106.71) (end 164.48 106.71) (width 1) (layer F.Cu) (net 57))
 (segment (start 167.64 100.33) (end 167.64 105.41) (width 1) (layer F.Cu) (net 57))
 (segment (start 167.64 105.41) (end 166.34 106.71) (width 1) (layer F.Cu) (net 57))
 (segment (start 153.6 119.38) (end 153.67 119.31) (width 1) (layer F.Cu) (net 57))
 (segment (start 144.46 120.92) (end 152.06 120.92) (width 1) (layer F.Cu) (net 57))
 (segment (start 152.06 120.92) (end 153.6 119.38) (width 1) (layer F.Cu) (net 57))
 (segment (start 163.83 93.98) (end 161.29 91.44) (width 1) (layer F.Cu) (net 57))
 (segment (start 167.64 93.98) (end 163.83 93.98) (width 1) (layer F.Cu) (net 57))
 (segment (start 161.29 91.44) (end 161.29 87.63) (width 1) (layer F.Cu) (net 57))
 (segment (start 165.1 85.09) (end 165.1 82.55) (width 1) (layer F.Cu) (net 57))
 (segment (start 163.83 86.36) (end 165.1 85.09) (width 1) (layer F.Cu) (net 57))
 (segment (start 155.01 120.65) (end 161.29 120.65) (width 1) (layer F.Cu) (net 57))
 (segment (start 161.29 120.65) (end 162.56 120.65) (width 1) (layer F.Cu) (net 57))
 (segment (start 161.29 87.63) (end 162.56 86.36) (width 1) (layer F.Cu) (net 57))
 (segment (start 162.56 86.36) (end 163.83 86.36) (width 1) (layer F.Cu) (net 57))
 (segment (start 163.83 88.9) (end 171.45 88.9) (width 1) (layer F.Cu) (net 61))
 (segment (start 132.805001 112.895001) (end 130.81 114.890002) (width 1) (layer F.Cu) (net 61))
 (segment (start 133.555001 112.895001) (end 132.805001 112.895001) (width 1) (layer F.Cu) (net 61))
 (segment (start 125.73 111.76) (end 121.92 111.76) (width 1) (layer F.Cu) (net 61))
 (segment (start 130.81 114.890002) (end 130.81 116.84) (width 1) (layer F.Cu) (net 61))
 (segment (start 125.73 114.3) (end 125.73 111.76) (width 1) (layer F.Cu) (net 61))
 (segment (start 130.81 116.84) (end 128.27 116.84) (width 1) (layer F.Cu) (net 61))
 (segment (start 128.27 116.84) (end 125.73 114.3) (width 1) (layer F.Cu) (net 61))
 (segment (start 138.43 121.92) (end 139.43 120.92) (width 1) (layer F.Cu) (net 61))
 (segment (start 142.56 120.92) (end 139.43 120.92) (width 1) (layer F.Cu) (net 61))
 (segment (start 134.62 121.92) (end 138.43 121.92) (width 1) (layer F.Cu) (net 61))
 (segment (start 130.81 116.84) (end 130.81 118.11) (width 1) (layer F.Cu) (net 61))
 (segment (start 130.81 118.11) (end 134.62 121.92) (width 1) (layer F.Cu) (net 61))
 (segment (start 168.91 115.57) (end 168.91 120.65) (width 1) (layer F.Cu) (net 61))
 (segment (start 171.45 88.9) (end 172.72 88.9) (width 1) (layer F.Cu) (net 61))
 (segment (start 172.72 88.9) (end 177.8 93.98) (width 1) (layer F.Cu) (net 61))
 (segment (start 177.8 93.98) (end 177.8 106.68) (width 1) (layer F.Cu) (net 61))
 (segment (start 177.8 106.68) (end 168.91 115.57) (width 1) (layer F.Cu) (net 61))
 (segment (start 166.37 123.19) (end 148.59 123.19) (width 1) (layer F.Cu) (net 61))
 (segment (start 168.91 120.65) (end 166.37 123.19) (width 1) (layer F.Cu) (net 61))
 (segment (start 148.59 125.73) (end 144.78 129.54) (width 1) (layer F.Cu) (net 61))
 (segment (start 148.59 123.19) (end 148.59 125.73) (width 1) (layer F.Cu) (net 61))
 (segment (start 138.43 121.92) (end 138.43 125.73) (width 1) (layer F.Cu) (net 61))
 (segment (start 142.24 129.54) (end 144.78 129.54) (width 1) (layer F.Cu) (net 61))
 (segment (start 138.43 125.73) (end 142.24 129.54) (width 1) (layer F.Cu) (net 61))
 (segment (start 120.65 111.76) (end 121.92 111.76) (width 1) (layer F.Cu) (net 61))
 (segment (start 143.51 125.73) (end 143.51 122.92) (width 1) (layer F.Cu) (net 56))
 (segment (start 161.29 110.49) (end 159.695001 108.895001) (width 1) (layer F.Cu) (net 60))
 (segment (start 166.694999 110.49) (end 161.29 110.49) (width 1) (layer F.Cu) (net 60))
 (segment (start 171.45 96.52) (end 171.45 105.734999) (width 1) (layer F.Cu) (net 60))
 (segment (start 171.45 105.734999) (end 166.694999 110.49) (width 1) (layer F.Cu) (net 60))
 (segment (start 159.695001 108.895001) (end 152.724999 108.895001) (width 1) (layer F.Cu) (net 60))
 (segment (start 154.615001 108.895001) (end 152.724999 108.895001) (width 1) (layer F.Cu) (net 60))
 (segment (start 152.724999 108.895001) (end 148.755001 108.895001) (width 1) (layer F.Cu) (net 60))
 (segment (start 148.755001 110.895001) (end 150.265001 110.895001) (width 0.25) (layer F.Cu) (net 62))
 (segment (start 161.29 113.03) (end 162.56 113.03) (width 1) (layer F.Cu) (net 62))
 (segment (start 148.755001 110.895001) (end 159.155001 110.895001) (width 1) (layer F.Cu) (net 62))
 (segment (start 159.155001 110.895001) (end 161.29 113.03) (width 1) (layer F.Cu) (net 62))
 (segment (start 133.555001 102.895001) (end 128.295001 102.895001) (width 1) (layer F.Cu) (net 63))
 (segment (start 128.295001 102.895001) (end 128.27 102.87) (width 1) (layer F.Cu) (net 63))
 (segment (start 128.295001 102.895001) (end 128.244999 102.895001) (width 1) (layer F.Cu) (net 63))
 (segment (start 163.83 96.52) (end 163.83 102.87) (width 1) (layer F.Cu) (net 58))
 (segment (start 164.48 103.52) (end 164.48 105.41) (width 1) (layer F.Cu) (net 58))
 (segment (start 163.83 102.87) (end 164.48 103.52) (width 1) (layer F.Cu) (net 58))
 (segment (start 161.074999 106.895001) (end 162.56 105.41) (width 1) (layer F.Cu) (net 58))
 (segment (start 153.835001 106.895001) (end 161.074999 106.895001) (width 1) (layer F.Cu) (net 58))
 (segment (start 162.56 105.41) (end 164.48 105.41) (width 1) (layer F.Cu) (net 58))
 (segment (start 153.835001 106.895001) (end 148.755001 106.895001) (width 1) (layer F.Cu) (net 58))
 (segment (start 133.555001 98.895001) (end 132.805001 98.895001) (width 1) (layer F.Cu) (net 59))
 (segment (start 132.805001 98.895001) (end 132.640002 99.06) (width 1) (layer F.Cu) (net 59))
 (segment (start 133.390002 99.06) (end 133.555001 98.895001) (width 1) (layer F.Cu) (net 59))
 (segment (start 133.555001 98.895001) (end 128.434999 98.895001) (width 1) (layer F.Cu) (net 59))
 (segment (start 126.059998 96.52) (end 128.434999 98.895001) (width 1) (layer F.Cu) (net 59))
 (segment (start 124.46 96.52) (end 126.059998 96.52) (width 1) (layer F.Cu) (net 59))
 (segment (start 124.46 88.9) (end 124.46 78.74) (width 1) (layer F.Cu) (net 9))
 (segment (start 123.19 77.47) (end 123.19 72.39) (width 1) (layer F.Cu) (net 9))
 (segment (start 124.46 78.74) (end 123.19 77.47) (width 1) (layer F.Cu) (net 9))
 (segment (start 132.99 100.33) (end 133.555001 100.895001) (width 1) (layer F.Cu) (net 55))
 (segment (start 129.54 100.33) (end 132.99 100.33) (width 1) (layer F.Cu) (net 55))
 (segment (start 136.155001 116.574999) (end 136.155001 114.395001) (width 1) (layer F.Cu) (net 54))
 (segment (start 134.62 118.11) (end 136.155001 116.574999) (width 1) (layer F.Cu) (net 54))
 (segment (start 138.155001 117.114999) (end 138.155001 114.395001) (width 1) (layer F.Cu) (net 53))
 (segment (start 137.16 118.11) (end 138.155001 117.114999) (width 1) (layer F.Cu) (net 53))
 (segment (start 140.155001 117.295001) (end 140.155001 114.395001) (width 1) (layer F.Cu) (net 52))
 (segment (start 140.97 118.11) (end 140.155001 117.295001) (width 1) (layer F.Cu) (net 52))
 (segment (start 142.24 114.48) (end 142.155001 114.395001) (width 1) (layer F.Cu) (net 51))
 (segment (start 142.155001 116.755001) (end 142.155001 114.395001) (width 1) (layer F.Cu) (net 51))
 (segment (start 143.51 118.11) (end 142.155001 116.755001) (width 1) (layer F.Cu) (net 51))
 (segment (start 144.155001 116.215001) (end 144.155001 114.395001) (width 1) (layer F.Cu) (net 50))
 (segment (start 146.05 118.11) (end 144.155001 116.215001) (width 1) (layer F.Cu) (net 50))
 (segment (start 148.59 118.11) (end 146.05 115.57) (width 1) (layer F.Cu) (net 49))
 (segment (start 146.155001 115.464999) (end 146.155001 114.395001) (width 1) (layer F.Cu) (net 49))
 (segment (start 146.05 115.57) (end 146.155001 115.464999) (width 1) (layer F.Cu) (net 49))
 (segment (start 132.8 104.14) (end 133.555001 104.895001) (width 1) (layer F.Cu) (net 48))
 (segment (start 129.54 104.14) (end 132.8 104.14) (width 1) (layer F.Cu) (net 48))
 (segment (start 133.34 106.68) (end 133.555001 106.895001) (width 1) (layer F.Cu) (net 47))
 (segment (start 129.54 106.68) (end 133.34 106.68) (width 1) (layer F.Cu) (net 47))
 (segment (start 133.230002 109.22) (end 133.555001 108.895001) (width 1) (layer F.Cu) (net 46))
 (segment (start 129.54 109.22) (end 133.230002 109.22) (width 1) (layer F.Cu) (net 46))
 (segment (start 130.404999 110.895001) (end 133.555001 110.895001) (width 1) (layer F.Cu) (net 45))
 (segment (start 129.54 111.76) (end 130.404999 110.895001) (width 1) (layer F.Cu) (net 45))
 (segment (start 149.27 105.41) (end 148.755001 104.895001) (width 1) (layer F.Cu) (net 44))
 (segment (start 152.4 105.41) (end 149.27 105.41) (width 1) (layer F.Cu) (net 44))
 (segment (start 148.780002 102.87) (end 148.755001 102.895001) (width 1) (layer F.Cu) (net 43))
 (segment (start 152.4 102.87) (end 148.780002 102.87) (width 1) (layer F.Cu) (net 43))
 (segment (start 159.865 83.975) (end 160.02 83.975) (width 1) (layer F.Cu) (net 2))
 (segment (start 160.02 82.55) (end 160.02 83.975) (width 1) (layer F.Cu) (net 2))
 (segment (start 150.564999 100.895001) (end 148.755001 100.895001) (width 1) (layer F.Cu) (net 2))
 (segment (start 155.644999 100.895001) (end 150.564999 100.895001) (width 1) (layer F.Cu) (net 2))
 (segment (start 158.75 97.79) (end 155.644999 100.895001) (width 1) (layer F.Cu) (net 2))
 (segment (start 158.75 86.36) (end 158.75 97.79) (width 1) (layer F.Cu) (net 2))
 (segment (start 160.02 83.975) (end 160.02 85.09) (width 1) (layer F.Cu) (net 2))
 (segment (start 160.02 85.09) (end 158.75 86.36) (width 1) (layer F.Cu) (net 2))
 (segment (start 151.294999 98.895001) (end 152.564999 98.895001) (width 1) (layer F.Cu) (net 1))
 (segment (start 148.755001 98.895001) (end 151.294999 98.895001) (width 1) (layer F.Cu) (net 1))
 (segment (start 152.564999 98.895001) (end 153.67 97.79) (width 1) (layer F.Cu) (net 1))
 (segment (start 154.94 96.52) (end 152.564999 98.895001) (width 1) (layer F.Cu) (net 1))
 (segment (start 154.94 82.55) (end 154.94 96.52) (width 1) (layer F.Cu) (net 1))
 (segment (start 124.46 100.33) (end 120.65 104.14) (width 1) (layer F.Cu) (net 59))
 (segment (start 124.46 96.52) (end 124.46 100.33) (width 1) (layer F.Cu) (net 59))
 (segment (start 125.73 104.14) (end 127 102.87) (width 1) (layer F.Cu) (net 63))
 (segment (start 127.025001 102.895001) (end 128.295001 102.895001) (width 1) (layer F.Cu) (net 63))
 (segment (start 127 102.87) (end 127.025001 102.895001) (width 1) (layer F.Cu) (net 63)))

